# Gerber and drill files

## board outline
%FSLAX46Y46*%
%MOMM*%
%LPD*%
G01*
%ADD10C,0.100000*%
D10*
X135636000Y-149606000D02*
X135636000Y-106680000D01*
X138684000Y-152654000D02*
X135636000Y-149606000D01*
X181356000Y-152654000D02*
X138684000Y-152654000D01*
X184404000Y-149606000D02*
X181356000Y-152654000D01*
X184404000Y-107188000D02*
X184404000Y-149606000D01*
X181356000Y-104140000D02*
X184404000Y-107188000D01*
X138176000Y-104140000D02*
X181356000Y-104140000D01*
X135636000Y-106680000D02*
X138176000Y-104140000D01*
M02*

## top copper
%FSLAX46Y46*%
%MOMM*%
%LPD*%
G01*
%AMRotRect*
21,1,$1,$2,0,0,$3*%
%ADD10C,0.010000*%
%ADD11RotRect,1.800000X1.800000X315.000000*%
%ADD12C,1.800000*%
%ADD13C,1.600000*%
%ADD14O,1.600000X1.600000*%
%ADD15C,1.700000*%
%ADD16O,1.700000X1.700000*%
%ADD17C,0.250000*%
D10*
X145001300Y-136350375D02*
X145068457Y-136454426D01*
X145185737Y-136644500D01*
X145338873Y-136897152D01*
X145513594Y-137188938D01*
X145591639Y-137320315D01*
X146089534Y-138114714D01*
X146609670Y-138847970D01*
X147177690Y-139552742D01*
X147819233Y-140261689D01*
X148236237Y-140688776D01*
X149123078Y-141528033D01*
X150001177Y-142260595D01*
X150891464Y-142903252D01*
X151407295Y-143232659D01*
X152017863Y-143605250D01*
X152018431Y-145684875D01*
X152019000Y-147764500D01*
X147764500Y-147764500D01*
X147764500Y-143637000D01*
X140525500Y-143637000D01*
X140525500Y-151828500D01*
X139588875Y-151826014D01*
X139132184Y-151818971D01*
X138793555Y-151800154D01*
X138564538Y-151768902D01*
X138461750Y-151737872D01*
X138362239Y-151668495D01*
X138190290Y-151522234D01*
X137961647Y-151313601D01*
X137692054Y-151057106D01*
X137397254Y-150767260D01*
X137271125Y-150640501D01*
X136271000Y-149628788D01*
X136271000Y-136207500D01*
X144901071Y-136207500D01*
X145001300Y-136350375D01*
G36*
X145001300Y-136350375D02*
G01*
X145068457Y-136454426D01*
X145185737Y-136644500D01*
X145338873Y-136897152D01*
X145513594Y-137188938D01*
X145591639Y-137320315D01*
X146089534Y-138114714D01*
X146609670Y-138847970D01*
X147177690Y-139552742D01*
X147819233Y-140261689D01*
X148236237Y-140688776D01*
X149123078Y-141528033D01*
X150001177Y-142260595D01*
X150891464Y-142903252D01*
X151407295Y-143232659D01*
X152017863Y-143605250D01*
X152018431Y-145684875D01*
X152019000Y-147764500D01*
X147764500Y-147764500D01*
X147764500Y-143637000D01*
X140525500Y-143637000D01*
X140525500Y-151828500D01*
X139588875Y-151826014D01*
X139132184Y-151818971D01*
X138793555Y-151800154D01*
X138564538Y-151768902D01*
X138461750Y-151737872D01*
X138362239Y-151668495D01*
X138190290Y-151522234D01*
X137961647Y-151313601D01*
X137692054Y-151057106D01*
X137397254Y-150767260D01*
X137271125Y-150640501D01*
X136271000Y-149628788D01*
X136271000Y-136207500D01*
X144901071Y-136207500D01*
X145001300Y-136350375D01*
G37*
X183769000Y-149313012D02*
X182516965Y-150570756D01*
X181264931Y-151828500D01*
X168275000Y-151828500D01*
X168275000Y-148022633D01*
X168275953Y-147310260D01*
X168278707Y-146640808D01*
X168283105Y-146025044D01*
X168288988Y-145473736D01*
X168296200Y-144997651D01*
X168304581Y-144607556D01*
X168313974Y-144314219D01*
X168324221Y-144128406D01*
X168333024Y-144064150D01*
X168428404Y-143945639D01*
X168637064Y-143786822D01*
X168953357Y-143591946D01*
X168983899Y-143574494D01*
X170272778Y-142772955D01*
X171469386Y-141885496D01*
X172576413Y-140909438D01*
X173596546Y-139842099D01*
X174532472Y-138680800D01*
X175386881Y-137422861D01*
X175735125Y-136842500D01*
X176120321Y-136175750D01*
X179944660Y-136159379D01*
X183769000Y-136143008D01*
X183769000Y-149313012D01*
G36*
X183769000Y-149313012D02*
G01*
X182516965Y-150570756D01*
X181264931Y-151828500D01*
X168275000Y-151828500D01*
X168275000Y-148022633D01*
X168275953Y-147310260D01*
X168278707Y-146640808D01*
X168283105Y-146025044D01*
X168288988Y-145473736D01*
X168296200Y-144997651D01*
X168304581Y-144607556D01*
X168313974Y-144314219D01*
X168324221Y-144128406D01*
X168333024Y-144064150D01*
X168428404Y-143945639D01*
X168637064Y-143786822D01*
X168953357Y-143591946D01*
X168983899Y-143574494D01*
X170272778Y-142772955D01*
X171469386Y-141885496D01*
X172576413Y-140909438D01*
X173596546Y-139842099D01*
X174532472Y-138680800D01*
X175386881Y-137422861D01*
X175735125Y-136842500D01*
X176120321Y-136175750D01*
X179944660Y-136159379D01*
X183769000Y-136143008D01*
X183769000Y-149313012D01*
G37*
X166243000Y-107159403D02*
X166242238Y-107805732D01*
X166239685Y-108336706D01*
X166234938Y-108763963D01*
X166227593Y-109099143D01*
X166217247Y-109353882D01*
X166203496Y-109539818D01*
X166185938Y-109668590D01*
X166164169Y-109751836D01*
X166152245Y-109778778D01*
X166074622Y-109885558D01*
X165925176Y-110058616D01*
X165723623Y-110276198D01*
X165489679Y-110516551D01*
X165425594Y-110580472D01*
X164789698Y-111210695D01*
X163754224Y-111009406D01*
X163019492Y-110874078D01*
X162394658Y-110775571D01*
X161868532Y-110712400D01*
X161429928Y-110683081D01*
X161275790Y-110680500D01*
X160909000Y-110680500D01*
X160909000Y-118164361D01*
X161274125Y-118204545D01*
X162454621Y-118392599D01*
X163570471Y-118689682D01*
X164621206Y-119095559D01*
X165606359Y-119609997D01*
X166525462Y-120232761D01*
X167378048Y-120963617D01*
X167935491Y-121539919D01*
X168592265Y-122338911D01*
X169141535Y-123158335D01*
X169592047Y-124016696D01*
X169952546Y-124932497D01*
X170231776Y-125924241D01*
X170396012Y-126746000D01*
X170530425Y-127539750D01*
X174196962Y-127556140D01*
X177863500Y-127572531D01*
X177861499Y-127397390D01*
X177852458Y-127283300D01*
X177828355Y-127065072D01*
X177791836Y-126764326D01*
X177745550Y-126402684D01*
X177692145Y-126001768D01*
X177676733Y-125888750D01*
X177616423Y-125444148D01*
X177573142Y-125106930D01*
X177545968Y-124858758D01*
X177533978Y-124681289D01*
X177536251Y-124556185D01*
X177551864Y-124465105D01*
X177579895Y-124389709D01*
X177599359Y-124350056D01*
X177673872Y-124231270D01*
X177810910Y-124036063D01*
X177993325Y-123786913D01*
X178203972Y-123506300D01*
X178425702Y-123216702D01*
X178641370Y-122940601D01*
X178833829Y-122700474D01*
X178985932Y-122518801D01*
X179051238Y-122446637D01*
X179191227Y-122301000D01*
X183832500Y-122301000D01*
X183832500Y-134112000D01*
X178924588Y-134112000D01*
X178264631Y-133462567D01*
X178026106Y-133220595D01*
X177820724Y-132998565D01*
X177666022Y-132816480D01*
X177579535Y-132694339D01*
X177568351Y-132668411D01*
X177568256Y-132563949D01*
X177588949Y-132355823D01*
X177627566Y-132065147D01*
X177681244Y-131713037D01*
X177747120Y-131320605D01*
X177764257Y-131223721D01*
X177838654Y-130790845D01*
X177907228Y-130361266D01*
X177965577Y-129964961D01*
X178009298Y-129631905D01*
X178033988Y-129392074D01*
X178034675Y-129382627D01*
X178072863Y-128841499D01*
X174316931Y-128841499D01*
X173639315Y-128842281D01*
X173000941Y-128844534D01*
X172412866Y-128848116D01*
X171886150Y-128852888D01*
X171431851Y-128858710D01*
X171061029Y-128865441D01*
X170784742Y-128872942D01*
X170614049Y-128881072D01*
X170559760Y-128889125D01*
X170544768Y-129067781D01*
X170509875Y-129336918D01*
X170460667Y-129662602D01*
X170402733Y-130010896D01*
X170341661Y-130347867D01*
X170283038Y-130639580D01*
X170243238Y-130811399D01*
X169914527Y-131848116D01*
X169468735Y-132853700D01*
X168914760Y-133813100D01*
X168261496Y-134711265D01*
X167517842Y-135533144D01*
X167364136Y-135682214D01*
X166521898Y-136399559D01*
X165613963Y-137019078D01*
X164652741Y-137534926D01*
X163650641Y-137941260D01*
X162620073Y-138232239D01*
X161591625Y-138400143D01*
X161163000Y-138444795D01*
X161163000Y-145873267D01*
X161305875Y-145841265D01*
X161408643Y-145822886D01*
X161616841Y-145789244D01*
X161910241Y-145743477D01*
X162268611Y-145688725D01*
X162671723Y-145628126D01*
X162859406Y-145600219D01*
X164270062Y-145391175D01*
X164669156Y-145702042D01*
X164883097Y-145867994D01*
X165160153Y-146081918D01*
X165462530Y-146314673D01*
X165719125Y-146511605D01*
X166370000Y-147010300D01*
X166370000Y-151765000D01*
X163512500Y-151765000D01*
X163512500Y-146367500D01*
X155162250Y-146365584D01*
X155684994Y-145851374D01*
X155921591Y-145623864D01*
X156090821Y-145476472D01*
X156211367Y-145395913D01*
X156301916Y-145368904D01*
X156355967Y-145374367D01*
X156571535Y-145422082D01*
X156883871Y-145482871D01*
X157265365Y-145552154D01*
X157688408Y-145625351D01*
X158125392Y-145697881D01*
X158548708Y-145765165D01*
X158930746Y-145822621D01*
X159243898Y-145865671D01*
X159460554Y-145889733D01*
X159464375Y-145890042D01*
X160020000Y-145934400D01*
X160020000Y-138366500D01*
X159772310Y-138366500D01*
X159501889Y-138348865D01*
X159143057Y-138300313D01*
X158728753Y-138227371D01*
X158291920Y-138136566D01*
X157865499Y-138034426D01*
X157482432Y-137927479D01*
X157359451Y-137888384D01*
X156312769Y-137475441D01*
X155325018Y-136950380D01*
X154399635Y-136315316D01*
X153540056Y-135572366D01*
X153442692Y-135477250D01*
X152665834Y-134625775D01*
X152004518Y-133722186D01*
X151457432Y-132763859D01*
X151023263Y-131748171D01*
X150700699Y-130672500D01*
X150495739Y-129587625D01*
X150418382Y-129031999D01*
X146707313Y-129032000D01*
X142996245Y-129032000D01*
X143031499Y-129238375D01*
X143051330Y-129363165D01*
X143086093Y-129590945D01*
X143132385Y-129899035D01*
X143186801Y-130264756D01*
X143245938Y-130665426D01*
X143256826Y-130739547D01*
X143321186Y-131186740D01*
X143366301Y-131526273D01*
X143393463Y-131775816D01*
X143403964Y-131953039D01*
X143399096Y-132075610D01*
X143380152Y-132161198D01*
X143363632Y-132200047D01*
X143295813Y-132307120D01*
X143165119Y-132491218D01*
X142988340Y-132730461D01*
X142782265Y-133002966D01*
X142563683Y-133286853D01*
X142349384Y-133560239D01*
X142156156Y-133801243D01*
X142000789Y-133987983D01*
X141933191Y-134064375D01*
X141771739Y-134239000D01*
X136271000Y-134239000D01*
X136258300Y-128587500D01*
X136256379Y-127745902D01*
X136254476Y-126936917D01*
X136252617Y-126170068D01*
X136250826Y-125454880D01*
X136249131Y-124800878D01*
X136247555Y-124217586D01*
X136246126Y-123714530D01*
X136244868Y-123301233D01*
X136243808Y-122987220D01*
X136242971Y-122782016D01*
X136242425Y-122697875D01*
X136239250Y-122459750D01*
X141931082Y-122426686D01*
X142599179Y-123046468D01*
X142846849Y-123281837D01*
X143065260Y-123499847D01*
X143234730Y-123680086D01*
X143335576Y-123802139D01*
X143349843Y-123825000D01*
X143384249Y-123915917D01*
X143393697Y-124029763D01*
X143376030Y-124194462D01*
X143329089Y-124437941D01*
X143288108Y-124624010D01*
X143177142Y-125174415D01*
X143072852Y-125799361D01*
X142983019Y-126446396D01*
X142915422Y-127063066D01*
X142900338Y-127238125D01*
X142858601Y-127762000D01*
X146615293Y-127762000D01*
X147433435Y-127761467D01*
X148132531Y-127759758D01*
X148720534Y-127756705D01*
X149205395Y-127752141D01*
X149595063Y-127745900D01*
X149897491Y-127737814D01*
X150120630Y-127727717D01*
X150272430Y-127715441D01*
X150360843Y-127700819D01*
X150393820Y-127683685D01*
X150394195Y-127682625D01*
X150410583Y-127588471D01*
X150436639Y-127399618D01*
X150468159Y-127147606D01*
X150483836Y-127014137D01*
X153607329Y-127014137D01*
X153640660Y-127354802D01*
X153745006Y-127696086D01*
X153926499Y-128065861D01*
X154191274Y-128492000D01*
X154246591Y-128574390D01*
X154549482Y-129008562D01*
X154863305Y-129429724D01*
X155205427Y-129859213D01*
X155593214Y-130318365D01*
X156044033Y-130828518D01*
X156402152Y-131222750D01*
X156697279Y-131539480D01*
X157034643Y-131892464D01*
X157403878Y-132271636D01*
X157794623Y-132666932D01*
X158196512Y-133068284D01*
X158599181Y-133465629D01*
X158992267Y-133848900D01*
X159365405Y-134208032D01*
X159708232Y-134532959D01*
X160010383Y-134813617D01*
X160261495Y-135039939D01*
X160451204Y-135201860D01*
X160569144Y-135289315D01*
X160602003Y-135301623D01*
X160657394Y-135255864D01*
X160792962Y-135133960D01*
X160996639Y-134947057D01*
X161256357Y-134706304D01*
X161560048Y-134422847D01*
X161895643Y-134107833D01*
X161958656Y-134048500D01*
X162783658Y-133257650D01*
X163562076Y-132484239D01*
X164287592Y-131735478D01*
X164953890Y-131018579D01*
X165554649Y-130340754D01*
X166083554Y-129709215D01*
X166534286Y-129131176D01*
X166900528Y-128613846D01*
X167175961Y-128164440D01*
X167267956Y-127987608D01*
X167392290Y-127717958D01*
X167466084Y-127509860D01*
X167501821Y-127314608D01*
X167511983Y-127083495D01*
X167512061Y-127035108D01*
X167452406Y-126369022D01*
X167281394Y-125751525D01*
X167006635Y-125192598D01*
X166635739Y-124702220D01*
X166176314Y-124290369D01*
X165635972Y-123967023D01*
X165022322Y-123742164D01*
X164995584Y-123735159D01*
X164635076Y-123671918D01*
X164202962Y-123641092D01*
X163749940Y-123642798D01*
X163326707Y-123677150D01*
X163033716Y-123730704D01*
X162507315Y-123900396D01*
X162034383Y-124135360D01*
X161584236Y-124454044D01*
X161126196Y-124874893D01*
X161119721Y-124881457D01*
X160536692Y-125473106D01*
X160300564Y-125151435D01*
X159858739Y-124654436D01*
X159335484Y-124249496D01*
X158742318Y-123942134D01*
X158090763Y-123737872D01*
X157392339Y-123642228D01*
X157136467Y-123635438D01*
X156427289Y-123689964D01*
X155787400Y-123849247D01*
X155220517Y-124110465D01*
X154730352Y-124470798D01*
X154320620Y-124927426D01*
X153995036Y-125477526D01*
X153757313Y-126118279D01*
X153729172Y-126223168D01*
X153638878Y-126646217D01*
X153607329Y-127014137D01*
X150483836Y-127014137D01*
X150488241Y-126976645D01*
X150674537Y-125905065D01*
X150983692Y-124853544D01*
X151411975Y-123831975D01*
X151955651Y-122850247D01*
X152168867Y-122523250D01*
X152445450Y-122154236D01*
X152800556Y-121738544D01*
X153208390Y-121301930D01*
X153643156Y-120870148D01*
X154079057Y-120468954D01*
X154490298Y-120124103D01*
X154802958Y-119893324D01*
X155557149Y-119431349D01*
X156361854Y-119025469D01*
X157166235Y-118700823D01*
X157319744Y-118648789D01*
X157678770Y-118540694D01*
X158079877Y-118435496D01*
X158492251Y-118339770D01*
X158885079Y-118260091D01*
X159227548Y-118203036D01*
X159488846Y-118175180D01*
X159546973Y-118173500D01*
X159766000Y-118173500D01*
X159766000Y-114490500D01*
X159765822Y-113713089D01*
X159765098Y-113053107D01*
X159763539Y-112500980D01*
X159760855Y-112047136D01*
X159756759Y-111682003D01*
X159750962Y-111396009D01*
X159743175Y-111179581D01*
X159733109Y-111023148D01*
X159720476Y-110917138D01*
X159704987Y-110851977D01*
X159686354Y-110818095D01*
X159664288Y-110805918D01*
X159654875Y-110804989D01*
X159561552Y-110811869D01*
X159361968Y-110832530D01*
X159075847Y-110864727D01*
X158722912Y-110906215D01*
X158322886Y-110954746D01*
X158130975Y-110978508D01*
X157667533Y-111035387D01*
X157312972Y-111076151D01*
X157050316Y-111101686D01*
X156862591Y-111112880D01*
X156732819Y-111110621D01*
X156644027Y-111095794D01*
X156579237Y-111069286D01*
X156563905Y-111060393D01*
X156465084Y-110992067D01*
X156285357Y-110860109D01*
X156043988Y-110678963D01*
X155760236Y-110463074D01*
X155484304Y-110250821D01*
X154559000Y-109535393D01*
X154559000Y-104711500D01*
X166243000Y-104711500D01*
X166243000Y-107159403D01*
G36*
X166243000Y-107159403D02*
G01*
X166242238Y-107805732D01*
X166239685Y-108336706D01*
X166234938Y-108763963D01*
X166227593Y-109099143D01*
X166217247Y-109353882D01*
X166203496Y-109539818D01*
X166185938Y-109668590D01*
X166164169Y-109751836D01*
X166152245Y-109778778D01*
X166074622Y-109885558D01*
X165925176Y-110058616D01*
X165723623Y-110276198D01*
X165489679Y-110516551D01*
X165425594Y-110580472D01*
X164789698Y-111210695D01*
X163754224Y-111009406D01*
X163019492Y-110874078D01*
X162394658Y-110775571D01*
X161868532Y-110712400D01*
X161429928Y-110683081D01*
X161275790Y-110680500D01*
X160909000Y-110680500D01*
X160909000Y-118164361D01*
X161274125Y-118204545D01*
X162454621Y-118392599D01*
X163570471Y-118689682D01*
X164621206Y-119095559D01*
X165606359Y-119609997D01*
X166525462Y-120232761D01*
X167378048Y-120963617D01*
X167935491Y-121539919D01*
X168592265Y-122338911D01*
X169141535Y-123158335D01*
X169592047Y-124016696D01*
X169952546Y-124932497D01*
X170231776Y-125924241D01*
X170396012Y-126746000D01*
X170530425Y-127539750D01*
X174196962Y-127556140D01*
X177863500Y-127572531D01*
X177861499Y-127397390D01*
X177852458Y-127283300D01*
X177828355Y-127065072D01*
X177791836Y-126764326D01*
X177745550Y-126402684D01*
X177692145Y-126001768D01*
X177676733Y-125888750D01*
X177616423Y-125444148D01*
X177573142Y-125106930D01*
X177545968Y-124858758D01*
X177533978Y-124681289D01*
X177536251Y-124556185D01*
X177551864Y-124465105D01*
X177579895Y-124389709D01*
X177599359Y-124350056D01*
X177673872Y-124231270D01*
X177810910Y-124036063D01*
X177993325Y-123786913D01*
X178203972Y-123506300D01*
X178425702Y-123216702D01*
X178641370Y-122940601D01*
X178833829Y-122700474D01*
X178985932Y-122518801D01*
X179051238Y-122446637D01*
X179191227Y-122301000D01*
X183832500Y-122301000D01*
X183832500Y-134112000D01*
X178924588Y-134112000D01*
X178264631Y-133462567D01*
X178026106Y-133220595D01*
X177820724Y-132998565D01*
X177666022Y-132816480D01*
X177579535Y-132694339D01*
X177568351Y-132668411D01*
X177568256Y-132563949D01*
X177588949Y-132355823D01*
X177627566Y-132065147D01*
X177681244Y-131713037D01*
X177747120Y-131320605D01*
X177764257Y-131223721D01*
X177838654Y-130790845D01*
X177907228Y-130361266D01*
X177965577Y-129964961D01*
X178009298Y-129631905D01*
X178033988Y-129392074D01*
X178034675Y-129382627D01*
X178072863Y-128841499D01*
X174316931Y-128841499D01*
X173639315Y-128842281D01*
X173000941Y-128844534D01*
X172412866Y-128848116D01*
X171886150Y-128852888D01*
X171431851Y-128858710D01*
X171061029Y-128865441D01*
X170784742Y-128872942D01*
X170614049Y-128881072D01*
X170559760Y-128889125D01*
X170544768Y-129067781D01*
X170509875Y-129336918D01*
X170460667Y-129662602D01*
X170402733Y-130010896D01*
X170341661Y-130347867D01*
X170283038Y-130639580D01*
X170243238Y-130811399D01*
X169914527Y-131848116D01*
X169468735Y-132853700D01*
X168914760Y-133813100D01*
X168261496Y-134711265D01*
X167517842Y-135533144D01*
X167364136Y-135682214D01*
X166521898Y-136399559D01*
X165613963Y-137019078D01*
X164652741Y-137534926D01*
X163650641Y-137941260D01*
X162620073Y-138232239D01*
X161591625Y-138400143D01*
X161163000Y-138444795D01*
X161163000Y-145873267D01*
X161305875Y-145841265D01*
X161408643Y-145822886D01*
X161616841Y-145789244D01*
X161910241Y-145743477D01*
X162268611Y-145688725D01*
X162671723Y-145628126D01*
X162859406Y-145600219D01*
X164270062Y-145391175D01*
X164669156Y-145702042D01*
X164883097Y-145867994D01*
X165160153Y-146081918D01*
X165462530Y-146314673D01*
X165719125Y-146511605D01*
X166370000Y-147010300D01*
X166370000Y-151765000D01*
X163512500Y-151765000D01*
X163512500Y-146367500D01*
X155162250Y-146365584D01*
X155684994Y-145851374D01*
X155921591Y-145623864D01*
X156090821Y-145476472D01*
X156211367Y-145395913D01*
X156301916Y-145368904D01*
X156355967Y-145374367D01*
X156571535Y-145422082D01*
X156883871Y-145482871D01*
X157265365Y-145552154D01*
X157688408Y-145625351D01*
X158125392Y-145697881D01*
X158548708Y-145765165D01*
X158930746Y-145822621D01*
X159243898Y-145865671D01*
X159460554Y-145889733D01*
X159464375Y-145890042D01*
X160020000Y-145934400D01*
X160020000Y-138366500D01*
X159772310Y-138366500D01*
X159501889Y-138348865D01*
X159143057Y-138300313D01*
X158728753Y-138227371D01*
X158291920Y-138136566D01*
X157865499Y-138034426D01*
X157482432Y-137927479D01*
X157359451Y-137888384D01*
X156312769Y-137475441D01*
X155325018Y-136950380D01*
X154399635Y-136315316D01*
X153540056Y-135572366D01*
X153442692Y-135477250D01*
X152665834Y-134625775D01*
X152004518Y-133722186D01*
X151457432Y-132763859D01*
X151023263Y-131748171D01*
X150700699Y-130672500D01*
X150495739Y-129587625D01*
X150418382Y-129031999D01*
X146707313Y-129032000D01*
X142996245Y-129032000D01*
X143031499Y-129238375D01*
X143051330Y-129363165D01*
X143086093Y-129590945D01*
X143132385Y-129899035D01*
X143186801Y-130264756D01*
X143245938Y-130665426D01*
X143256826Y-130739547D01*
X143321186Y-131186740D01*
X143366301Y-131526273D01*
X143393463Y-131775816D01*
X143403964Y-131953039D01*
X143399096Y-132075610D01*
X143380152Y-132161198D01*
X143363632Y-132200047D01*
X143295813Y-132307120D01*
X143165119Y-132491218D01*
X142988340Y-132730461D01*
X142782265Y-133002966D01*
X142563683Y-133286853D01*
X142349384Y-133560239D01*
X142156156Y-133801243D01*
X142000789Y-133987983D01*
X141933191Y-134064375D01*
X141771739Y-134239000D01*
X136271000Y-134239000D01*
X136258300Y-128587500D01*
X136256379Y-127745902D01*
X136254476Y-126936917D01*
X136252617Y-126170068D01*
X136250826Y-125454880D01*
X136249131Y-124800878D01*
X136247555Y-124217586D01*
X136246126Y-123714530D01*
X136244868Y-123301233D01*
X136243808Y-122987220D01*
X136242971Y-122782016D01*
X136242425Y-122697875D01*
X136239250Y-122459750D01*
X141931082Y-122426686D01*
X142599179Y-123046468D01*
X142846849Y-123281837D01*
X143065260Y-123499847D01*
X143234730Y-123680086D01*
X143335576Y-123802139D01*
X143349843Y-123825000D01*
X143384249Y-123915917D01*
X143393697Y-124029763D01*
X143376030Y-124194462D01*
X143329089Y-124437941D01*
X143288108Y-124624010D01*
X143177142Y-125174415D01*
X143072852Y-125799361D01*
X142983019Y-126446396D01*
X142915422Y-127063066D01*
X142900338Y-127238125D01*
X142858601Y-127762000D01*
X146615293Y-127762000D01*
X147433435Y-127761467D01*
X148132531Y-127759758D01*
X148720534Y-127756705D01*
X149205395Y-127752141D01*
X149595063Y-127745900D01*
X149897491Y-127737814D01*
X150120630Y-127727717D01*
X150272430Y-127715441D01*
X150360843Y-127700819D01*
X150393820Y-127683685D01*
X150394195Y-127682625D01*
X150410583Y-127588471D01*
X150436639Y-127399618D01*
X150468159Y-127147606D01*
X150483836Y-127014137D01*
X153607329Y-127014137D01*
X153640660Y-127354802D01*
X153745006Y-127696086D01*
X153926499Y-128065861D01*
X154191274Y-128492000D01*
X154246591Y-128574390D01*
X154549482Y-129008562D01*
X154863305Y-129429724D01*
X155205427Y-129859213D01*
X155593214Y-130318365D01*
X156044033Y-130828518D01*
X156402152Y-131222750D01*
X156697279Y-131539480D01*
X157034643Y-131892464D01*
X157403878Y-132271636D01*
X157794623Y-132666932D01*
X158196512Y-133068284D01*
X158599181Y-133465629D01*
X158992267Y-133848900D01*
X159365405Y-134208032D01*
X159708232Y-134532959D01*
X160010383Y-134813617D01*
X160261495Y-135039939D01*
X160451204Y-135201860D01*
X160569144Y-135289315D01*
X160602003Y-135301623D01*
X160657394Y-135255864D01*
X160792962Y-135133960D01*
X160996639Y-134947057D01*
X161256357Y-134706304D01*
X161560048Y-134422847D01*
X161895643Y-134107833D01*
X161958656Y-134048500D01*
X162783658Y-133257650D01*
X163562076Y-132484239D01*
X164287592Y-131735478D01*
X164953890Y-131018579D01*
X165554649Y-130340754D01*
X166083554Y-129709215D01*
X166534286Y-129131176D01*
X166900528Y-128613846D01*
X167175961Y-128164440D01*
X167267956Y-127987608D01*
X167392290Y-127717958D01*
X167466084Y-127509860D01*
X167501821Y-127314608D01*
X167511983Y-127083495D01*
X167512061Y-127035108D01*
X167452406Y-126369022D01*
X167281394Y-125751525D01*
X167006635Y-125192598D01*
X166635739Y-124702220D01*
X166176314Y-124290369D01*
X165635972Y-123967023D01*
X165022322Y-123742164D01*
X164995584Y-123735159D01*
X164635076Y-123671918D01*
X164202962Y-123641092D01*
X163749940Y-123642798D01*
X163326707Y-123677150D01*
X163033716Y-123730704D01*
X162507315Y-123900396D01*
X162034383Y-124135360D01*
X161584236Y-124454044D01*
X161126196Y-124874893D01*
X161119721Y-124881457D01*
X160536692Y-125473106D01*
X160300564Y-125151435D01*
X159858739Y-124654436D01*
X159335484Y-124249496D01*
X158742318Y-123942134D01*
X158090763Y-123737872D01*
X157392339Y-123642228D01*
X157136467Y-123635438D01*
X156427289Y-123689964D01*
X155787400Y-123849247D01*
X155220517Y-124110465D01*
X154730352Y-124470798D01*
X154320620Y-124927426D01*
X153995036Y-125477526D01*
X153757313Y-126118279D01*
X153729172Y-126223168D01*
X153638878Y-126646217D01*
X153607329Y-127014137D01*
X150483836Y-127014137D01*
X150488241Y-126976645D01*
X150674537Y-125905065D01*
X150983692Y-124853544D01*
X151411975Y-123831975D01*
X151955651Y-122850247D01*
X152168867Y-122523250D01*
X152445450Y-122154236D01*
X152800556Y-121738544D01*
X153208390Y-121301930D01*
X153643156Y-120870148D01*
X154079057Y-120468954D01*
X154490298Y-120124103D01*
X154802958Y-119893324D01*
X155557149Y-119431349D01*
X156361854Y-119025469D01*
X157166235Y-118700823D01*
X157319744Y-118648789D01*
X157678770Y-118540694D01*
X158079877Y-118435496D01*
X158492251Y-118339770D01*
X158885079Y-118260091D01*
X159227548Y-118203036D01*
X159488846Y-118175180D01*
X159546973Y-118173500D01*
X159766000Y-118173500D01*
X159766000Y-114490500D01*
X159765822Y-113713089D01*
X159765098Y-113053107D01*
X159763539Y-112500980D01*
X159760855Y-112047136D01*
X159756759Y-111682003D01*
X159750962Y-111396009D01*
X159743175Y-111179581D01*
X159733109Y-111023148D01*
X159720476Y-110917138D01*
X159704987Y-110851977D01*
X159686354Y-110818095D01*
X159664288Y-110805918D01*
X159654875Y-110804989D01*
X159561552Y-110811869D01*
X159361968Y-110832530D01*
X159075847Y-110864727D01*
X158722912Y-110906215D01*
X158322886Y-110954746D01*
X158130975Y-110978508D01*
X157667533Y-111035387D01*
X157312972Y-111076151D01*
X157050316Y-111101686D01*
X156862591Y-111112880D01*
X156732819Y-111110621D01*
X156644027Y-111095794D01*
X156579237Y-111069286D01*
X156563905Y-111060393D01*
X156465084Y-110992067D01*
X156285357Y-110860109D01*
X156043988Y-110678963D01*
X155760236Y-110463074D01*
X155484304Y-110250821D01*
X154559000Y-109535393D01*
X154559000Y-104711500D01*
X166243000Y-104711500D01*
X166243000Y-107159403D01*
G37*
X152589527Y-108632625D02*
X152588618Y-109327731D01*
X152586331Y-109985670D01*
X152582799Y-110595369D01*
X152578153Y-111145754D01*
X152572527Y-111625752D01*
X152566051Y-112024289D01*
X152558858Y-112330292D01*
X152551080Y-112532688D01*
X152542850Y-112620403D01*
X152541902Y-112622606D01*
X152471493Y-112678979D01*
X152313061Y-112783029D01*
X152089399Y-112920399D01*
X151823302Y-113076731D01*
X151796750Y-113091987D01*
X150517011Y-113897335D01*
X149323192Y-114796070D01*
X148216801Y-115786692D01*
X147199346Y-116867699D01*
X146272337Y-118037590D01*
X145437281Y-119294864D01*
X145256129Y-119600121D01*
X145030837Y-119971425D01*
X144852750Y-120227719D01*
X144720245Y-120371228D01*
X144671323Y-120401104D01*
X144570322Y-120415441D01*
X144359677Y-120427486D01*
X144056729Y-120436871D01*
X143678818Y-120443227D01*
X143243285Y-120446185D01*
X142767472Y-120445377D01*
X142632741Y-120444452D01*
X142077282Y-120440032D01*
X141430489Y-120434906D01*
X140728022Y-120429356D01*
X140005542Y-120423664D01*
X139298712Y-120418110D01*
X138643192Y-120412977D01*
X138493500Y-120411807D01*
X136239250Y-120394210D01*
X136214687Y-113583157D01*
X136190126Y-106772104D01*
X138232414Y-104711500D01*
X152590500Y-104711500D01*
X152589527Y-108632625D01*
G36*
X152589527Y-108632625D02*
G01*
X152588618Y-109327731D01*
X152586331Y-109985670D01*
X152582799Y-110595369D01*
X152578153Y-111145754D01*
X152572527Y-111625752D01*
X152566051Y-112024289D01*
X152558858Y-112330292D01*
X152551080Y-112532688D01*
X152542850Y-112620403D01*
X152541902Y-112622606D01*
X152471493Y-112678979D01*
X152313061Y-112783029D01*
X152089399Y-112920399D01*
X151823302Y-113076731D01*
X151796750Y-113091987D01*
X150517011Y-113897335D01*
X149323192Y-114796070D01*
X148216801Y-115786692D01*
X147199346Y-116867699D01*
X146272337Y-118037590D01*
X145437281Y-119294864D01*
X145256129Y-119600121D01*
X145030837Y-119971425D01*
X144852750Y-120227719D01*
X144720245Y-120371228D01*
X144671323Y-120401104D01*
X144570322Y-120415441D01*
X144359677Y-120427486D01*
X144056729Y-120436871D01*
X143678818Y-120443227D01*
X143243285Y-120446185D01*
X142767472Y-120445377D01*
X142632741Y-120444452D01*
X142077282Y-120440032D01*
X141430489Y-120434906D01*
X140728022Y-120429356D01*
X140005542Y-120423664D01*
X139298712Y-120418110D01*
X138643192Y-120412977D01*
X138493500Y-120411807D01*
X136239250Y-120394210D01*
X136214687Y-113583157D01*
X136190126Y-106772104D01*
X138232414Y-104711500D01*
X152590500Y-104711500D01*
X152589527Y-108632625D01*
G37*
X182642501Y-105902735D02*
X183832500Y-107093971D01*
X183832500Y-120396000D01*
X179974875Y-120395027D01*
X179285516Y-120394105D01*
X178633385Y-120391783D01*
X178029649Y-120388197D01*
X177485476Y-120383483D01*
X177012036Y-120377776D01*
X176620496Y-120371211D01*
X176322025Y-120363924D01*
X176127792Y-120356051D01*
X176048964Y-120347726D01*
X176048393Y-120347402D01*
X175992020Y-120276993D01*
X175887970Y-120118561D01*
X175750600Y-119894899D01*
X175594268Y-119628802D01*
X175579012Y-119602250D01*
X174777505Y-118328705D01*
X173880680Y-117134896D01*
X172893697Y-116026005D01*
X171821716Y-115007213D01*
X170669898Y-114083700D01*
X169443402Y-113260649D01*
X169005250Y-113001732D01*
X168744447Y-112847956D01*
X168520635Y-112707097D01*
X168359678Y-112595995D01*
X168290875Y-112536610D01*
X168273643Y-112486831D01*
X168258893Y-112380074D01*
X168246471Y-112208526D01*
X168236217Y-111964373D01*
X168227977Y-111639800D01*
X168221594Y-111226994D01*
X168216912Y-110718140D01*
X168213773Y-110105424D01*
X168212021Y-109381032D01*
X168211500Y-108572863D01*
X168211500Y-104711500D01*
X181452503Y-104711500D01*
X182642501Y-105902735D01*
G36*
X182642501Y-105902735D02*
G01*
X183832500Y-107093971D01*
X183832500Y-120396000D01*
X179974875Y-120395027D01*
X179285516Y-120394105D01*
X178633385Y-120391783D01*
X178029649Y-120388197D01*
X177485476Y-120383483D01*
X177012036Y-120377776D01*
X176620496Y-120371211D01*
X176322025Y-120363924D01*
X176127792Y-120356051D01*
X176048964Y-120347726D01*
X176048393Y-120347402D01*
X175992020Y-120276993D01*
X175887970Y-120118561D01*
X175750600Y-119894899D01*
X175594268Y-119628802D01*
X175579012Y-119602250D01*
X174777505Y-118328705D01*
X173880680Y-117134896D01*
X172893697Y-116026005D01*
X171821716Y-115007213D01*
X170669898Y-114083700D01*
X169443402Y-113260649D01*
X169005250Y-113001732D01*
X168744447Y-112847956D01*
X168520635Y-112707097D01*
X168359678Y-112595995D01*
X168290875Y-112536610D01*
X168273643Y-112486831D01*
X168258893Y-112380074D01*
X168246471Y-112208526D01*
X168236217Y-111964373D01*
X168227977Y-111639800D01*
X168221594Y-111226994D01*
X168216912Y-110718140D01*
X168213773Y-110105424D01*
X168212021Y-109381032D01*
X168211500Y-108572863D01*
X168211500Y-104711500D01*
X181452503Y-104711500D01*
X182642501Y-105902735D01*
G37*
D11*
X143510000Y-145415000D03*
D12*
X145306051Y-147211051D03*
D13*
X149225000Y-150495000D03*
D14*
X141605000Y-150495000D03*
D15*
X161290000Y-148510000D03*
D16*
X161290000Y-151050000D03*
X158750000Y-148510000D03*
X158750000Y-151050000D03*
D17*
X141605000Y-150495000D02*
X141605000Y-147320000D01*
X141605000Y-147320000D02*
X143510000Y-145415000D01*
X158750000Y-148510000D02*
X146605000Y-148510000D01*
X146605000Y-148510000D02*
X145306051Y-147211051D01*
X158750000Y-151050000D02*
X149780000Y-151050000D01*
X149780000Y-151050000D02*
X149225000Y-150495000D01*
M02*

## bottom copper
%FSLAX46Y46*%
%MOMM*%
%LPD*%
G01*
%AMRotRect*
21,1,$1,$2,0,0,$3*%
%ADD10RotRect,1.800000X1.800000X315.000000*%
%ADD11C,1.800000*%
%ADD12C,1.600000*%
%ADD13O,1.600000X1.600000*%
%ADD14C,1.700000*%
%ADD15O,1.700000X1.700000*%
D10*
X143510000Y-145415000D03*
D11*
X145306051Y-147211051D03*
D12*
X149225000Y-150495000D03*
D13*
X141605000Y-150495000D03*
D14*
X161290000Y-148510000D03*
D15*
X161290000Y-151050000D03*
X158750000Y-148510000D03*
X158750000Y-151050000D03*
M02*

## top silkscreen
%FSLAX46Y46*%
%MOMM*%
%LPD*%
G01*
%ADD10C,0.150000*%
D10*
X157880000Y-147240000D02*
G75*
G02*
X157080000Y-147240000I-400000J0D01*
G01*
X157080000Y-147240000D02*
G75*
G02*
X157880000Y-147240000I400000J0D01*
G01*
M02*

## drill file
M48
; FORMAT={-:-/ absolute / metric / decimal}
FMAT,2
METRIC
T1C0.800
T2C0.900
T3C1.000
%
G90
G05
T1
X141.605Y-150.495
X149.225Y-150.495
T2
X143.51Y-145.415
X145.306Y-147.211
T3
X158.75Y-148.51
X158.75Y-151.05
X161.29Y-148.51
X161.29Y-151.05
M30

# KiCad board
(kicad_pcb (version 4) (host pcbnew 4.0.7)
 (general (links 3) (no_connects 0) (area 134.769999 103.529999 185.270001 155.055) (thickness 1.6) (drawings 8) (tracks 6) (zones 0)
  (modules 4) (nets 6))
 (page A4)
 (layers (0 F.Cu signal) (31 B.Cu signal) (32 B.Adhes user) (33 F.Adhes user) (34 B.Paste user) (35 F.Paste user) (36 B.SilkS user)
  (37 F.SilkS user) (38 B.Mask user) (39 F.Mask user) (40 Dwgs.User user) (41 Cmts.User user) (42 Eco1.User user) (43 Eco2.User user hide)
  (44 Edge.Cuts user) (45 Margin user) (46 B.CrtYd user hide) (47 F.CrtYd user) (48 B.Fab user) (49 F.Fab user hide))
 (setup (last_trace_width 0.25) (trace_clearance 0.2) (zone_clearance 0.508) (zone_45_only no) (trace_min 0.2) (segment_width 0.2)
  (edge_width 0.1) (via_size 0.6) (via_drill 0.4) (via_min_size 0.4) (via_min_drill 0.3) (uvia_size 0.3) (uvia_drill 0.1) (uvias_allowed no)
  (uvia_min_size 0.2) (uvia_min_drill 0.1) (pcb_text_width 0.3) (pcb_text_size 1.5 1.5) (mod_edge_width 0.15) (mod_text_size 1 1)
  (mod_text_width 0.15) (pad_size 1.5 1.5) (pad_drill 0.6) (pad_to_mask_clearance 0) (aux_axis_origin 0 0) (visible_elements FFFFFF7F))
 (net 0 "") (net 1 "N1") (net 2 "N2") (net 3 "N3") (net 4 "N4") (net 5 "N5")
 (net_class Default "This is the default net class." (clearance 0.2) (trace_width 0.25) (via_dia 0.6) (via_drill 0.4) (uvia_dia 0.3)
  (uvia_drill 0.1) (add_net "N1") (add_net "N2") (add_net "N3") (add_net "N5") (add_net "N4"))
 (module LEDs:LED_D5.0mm (layer B.Cu) (at 143.51 145.415 315)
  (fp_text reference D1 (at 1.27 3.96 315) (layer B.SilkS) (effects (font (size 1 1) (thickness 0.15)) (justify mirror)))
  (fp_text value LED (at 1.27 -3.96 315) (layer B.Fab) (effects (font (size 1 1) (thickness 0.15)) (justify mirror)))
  (pad 1 thru_hole rect (at 0 0 315) (size 1.8 1.8) (drill 0.9) (layers *.Cu *.Mask) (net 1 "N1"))
  (pad 2 thru_hole circle (at 2.54 0 315) (size 1.8 1.8) (drill 0.9) (layers *.Cu *.Mask) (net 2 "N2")))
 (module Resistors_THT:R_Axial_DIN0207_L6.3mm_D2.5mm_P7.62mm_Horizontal (layer B.Cu) (at 149.225 150.495 180)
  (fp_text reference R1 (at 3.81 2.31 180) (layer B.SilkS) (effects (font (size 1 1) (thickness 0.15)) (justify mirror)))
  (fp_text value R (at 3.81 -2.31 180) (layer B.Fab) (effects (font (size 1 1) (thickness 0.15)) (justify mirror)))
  (pad 1 thru_hole circle (at 0 0 180) (size 1.6 1.6) (drill 0.8) (layers *.Cu *.Mask) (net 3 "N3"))
  (pad 2 thru_hole oval (at 7.62 0 180) (size 1.6 1.6) (drill 0.8) (layers *.Cu *.Mask) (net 1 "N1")))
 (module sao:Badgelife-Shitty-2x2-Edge (layer F.Cu) (at 160.02 144.78)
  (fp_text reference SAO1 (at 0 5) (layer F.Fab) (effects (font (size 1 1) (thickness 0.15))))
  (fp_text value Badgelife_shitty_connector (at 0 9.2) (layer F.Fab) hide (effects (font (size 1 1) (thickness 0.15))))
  (fp_circle (center -2.54 2.46) (end -2.14 2.46) (layer F.SilkS) (width 0.15))
  (pad 4 thru_hole circle (at 1.27 3.73) (size 1.7 1.7) (drill 1) (layers *.Cu *.Mask) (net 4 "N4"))
  (pad 3 thru_hole oval (at 1.27 6.27) (size 1.7 1.7) (drill 1) (layers *.Cu *.Mask) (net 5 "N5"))
  (pad 1 thru_hole oval (at -1.27 3.73) (size 1.7 1.7) (drill 1) (layers *.Cu *.Mask) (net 2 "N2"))
  (pad 2 thru_hole oval (at -1.27 6.27) (size 1.7 1.7) (drill 1) (layers *.Cu *.Mask) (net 3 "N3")))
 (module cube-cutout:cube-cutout (layer F.Cu) (at 160.02 128.27)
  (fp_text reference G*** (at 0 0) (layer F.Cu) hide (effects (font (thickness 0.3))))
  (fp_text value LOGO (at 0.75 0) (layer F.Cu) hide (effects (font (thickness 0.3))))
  (fp_poly
   (pts (xy -15.0187 8.080375) (xy -14.951543 8.184426) (xy -14.834263 8.3745) (xy -14.681127 8.627152) (xy -14.506406 8.918938)
    (xy -14.428361 9.050315) (xy -13.930466 9.844714) (xy -13.41033 10.57797) (xy -12.84231 11.282742) (xy -12.200767 11.991689)
    (xy -11.783763 12.418776) (xy -10.896922 13.258033) (xy -10.018823 13.990595) (xy -9.128536 14.633252) (xy -8.612705 14.962659)
    (xy -8.002137 15.33525) (xy -8.001569 17.414875) (xy -8.001 19.4945) (xy -12.2555 19.4945) (xy -12.2555 15.367) (xy -19.4945 15.367)
    (xy -19.4945 23.5585) (xy -20.431125 23.556014) (xy -20.887816 23.548971) (xy -21.226445 23.530154) (xy -21.455462 23.498902)
    (xy -21.55825 23.467872) (xy -21.657761 23.398495) (xy -21.82971 23.252234) (xy -22.058353 23.043601) (xy -22.327946 22.787106)
    (xy -22.622746 22.49726) (xy -22.748875 22.370501) (xy -23.749 21.358788) (xy -23.749 7.9375) (xy -15.118929 7.9375)
    (xy -15.0187 8.080375))
   (layer F.Cu) (width 0.01))
  (fp_poly
   (pts (xy 23.749 21.043012) (xy 22.496965 22.300756) (xy 21.244931 23.5585) (xy 8.255 23.5585) (xy 8.255 19.752633) (xy 8.255953 19.04026)
    (xy 8.258707 18.370808) (xy 8.263105 17.755044) (xy 8.268988 17.203736) (xy 8.2762 16.727651) (xy 8.284581 16.337556)
    (xy 8.293974 16.044219) (xy 8.304221 15.858406) (xy 8.313024 15.79415) (xy 8.408404 15.675639) (xy 8.617064 15.516822)
    (xy 8.933357 15.321946) (xy 8.963899 15.304494) (xy 10.252778 14.502955) (xy 11.449386 13.615496) (xy 12.556413 12.639438)
    (xy 13.576546 11.572099) (xy 14.512472 10.4108) (xy 15.366881 9.152861) (xy 15.715125 8.5725) (xy 16.100321 7.90575)
    (xy 19.92466 7.889379) (xy 23.749 7.873008) (xy 23.749 21.043012))
   (layer F.Cu) (width 0.01))
  (fp_poly
   (pts (xy 6.223 -21.110597) (xy 6.222238 -20.464268) (xy 6.219685 -19.933294) (xy 6.214938 -19.506037) (xy 6.207593 -19.170857)
    (xy 6.197247 -18.916118) (xy 6.183496 -18.730182) (xy 6.165938 -18.60141) (xy 6.144169 -18.518164) (xy 6.132245 -18.491222)
    (xy 6.054622 -18.384442) (xy 5.905176 -18.211384) (xy 5.703623 -17.993802) (xy 5.469679 -17.753449) (xy 5.405594 -17.689528)
    (xy 4.769698 -17.059305) (xy 3.734224 -17.260594) (xy 2.999492 -17.395922) (xy 2.374658 -17.494429) (xy 1.848532 -17.5576)
    (xy 1.409928 -17.586919) (xy 1.25579 -17.5895) (xy 0.889 -17.5895) (xy 0.889 -10.105639) (xy 1.254125 -10.065455)
    (xy 2.434621 -9.877401) (xy 3.550471 -9.580318) (xy 4.601206 -9.174441) (xy 5.586359 -8.660003) (xy 6.505462 -8.037239)
    (xy 7.358048 -7.306383) (xy 7.915491 -6.730081) (xy 8.572265 -5.931089) (xy 9.121535 -5.111665) (xy 9.572047 -4.253304)
    (xy 9.932546 -3.337503) (xy 10.211776 -2.345759) (xy 10.376012 -1.524) (xy 10.510425 -0.73025) (xy 14.176962 -0.71386)
    (xy 17.8435 -0.697469) (xy 17.841499 -0.87261) (xy 17.832458 -0.9867) (xy 17.808355 -1.204928) (xy 17.771836 -1.505674)
    (xy 17.72555 -1.867316) (xy 17.672145 -2.268232) (xy 17.656733 -2.38125) (xy 17.596423 -2.825852) (xy 17.553142 -3.16307)
    (xy 17.525968 -3.411242) (xy 17.513978 -3.588711) (xy 17.516251 -3.713815) (xy 17.531864 -3.804895) (xy 17.559895 -3.880291)
    (xy 17.579359 -3.919944) (xy 17.653872 -4.03873) (xy 17.79091 -4.233937) (xy 17.973325 -4.483087) (xy 18.183972 -4.7637)
    (xy 18.405702 -5.053298) (xy 18.62137 -5.329399) (xy 18.813829 -5.569526) (xy 18.965932 -5.751199) (xy 19.031238 -5.823363)
    (xy 19.171227 -5.969) (xy 23.8125 -5.969) (xy 23.8125 5.842) (xy 18.904588 5.842) (xy 18.244631 5.192567) (xy 18.006106 4.950595)
    (xy 17.800724 4.728565) (xy 17.646022 4.54648) (xy 17.559535 4.424339) (xy 17.548351 4.398411) (xy 17.548256 4.293949)
    (xy 17.568949 4.085823) (xy 17.607566 3.795147) (xy 17.661244 3.443037) (xy 17.72712 3.050605) (xy 17.744257 2.953721)
    (xy 17.818654 2.520845) (xy 17.887228 2.091266) (xy 17.945577 1.694961) (xy 17.989298 1.361905) (xy 18.013988 1.122074)
    (xy 18.014675 1.112627) (xy 18.052863 0.571499) (xy 14.296931 0.571499) (xy 13.619315 0.572281) (xy 12.980941 0.574534)
    (xy 12.392866 0.578116) (xy 11.86615 0.582888) (xy 11.411851 0.58871) (xy 11.041029 0.595441) (xy 10.764742 0.602942)
    (xy 10.594049 0.611072) (xy 10.53976 0.619125) (xy 10.524768 0.797781) (xy 10.489875 1.066918) (xy 10.440667 1.392602)
    (xy 10.382733 1.740896) (xy 10.321661 2.077867) (xy 10.263038 2.36958) (xy 10.223238 2.541399) (xy 9.894527 3.578116)
    (xy 9.448735 4.5837) (xy 8.89476 5.5431) (xy 8.241496 6.441265) (xy 7.497842 7.263144) (xy 7.344136 7.412214) (xy 6.501898 8.129559)
    (xy 5.593963 8.749078) (xy 4.632741 9.264926) (xy 3.630641 9.67126) (xy 2.600073 9.962239) (xy 1.571625 10.130143) (xy 1.143 10.174795)
    (xy 1.143 17.603267) (xy 1.285875 17.571265) (xy 1.388643 17.552886) (xy 1.596841 17.519244) (xy 1.890241 17.473477)
    (xy 2.248611 17.418725) (xy 2.651723 17.358126) (xy 2.839406 17.330219) (xy 4.250062 17.121175) (xy 4.649156 17.432042)
    (xy 4.863097 17.597994) (xy 5.140153 17.811918) (xy 5.44253 18.044673) (xy 5.699125 18.241605) (xy 6.35 18.7403) (xy 6.35 23.495)
    (xy 3.4925 23.495) (xy 3.4925 18.0975) (xy -4.85775 18.095584) (xy -4.335006 17.581374) (xy -4.098409 17.353864)
    (xy -3.929179 17.206472) (xy -3.808633 17.125913) (xy -3.718084 17.098904) (xy -3.664033 17.104367) (xy -3.448465 17.152082)
    (xy -3.136129 17.212871) (xy -2.754635 17.282154) (xy -2.331592 17.355351) (xy -1.894608 17.427881) (xy -1.471292 17.495165)
    (xy -1.089254 17.552621) (xy -0.776102 17.595671) (xy -0.559446 17.619733) (xy -0.555625 17.620042) (xy 0 17.6644) (xy 0 10.0965)
    (xy -0.24769 10.0965) (xy -0.518111 10.078865) (xy -0.876943 10.030313) (xy -1.291247 9.957371) (xy -1.72808 9.866566)
    (xy -2.154501 9.764426) (xy -2.537568 9.657479) (xy -2.660549 9.618384) (xy -3.707231 9.205441) (xy -4.694982 8.68038)
    (xy -5.620365 8.045316) (xy -6.479944 7.302366) (xy -6.577308 7.20725) (xy -7.354166 6.355775) (xy -8.015482 5.452186)
    (xy -8.562568 4.493859) (xy -8.996737 3.478171) (xy -9.319301 2.4025) (xy -9.524261 1.317625) (xy -9.601618 0.761999)
    (xy -13.312687 0.762) (xy -17.023755 0.762) (xy -16.988501 0.968375) (xy -16.96867 1.093165) (xy -16.933907 1.320945)
    (xy -16.887615 1.629035) (xy -16.833199 1.994756) (xy -16.774062 2.395426) (xy -16.763174 2.469547) (xy -16.698814 2.91674)
    (xy -16.653699 3.256273) (xy -16.626537 3.505816) (xy -16.616036 3.683039) (xy -16.620904 3.80561) (xy -16.639848 3.891198)
    (xy -16.656368 3.930047) (xy -16.724187 4.03712) (xy -16.854881 4.221218) (xy -17.03166 4.460461) (xy -17.237735 4.732966)
    (xy -17.456317 5.016853) (xy -17.670616 5.290239) (xy -17.863844 5.531243) (xy -18.019211 5.717983) (xy -18.086809 5.794375)
    (xy -18.248261 5.969) (xy -23.749 5.969) (xy -23.7617 0.3175) (xy -23.763621 -0.524098) (xy -23.765524 -1.333083)
    (xy -23.767383 -2.099932) (xy -23.769174 -2.81512) (xy -23.770869 -3.469122) (xy -23.772445 -4.052414) (xy -23.773874 -4.55547)
    (xy -23.775132 -4.968767) (xy -23.776192 -5.28278) (xy -23.777029 -5.487984) (xy -23.777575 -5.572125) (xy -23.78075 -5.81025)
    (xy -18.088918 -5.843314) (xy -17.420821 -5.223532) (xy -17.173151 -4.988163) (xy -16.95474 -4.770153) (xy -16.78527 -4.589914)
    (xy -16.684424 -4.467861) (xy -16.670157 -4.445) (xy -16.635751 -4.354083) (xy -16.626303 -4.240237) (xy -16.64397 -4.075538)
    (xy -16.690911 -3.832059) (xy -16.731892 -3.64599) (xy -16.842858 -3.095585) (xy -16.947148 -2.470639) (xy -17.036981 -1.823604)
    (xy -17.104578 -1.206934) (xy -17.119662 -1.031875) (xy -17.161399 -0.508) (xy -13.404707 -0.508) (xy -12.586565 -0.508533)
    (xy -11.887469 -0.510242) (xy -11.299466 -0.513295) (xy -10.814605 -0.517859) (xy -10.424937 -0.5241) (xy -10.122509 -0.532186)
    (xy -9.89937 -0.542283) (xy -9.74757 -0.554559) (xy -9.659157 -0.569181) (xy -9.62618 -0.586315) (xy -9.625805 -0.587375)
    (xy -9.609417 -0.681529) (xy -9.583361 -0.870382) (xy -9.551841 -1.122394) (xy -9.536164 -1.255863) (xy -6.412671 -1.255863)
    (xy -6.37934 -0.915198) (xy -6.274994 -0.573914) (xy -6.093501 -0.204139) (xy -5.828726 0.222) (xy -5.773409 0.30439)
    (xy -5.470518 0.738562) (xy -5.156695 1.159724) (xy -4.814573 1.589213) (xy -4.426786 2.048365) (xy -3.975967 2.558518)
    (xy -3.617848 2.95275) (xy -3.322721 3.26948) (xy -2.985357 3.622464) (xy -2.616122 4.001636) (xy -2.225377 4.396932)
    (xy -1.823488 4.798284) (xy -1.420819 5.195629) (xy -1.027733 5.5789) (xy -0.654595 5.938032) (xy -0.311768 6.262959)
    (xy -0.009617 6.543617) (xy 0.241495 6.769939) (xy 0.431204 6.93186) (xy 0.549144 7.019315) (xy 0.582003 7.031623)
    (xy 0.637394 6.985864) (xy 0.772962 6.86396) (xy 0.976639 6.677057) (xy 1.236357 6.436304) (xy 1.540048 6.152847) (xy 1.875643 5.837833)
    (xy 1.938656 5.7785) (xy 2.763658 4.98765) (xy 3.542076 4.214239) (xy 4.267592 3.465478) (xy 4.93389 2.748579) (xy 5.534649 2.070754)
    (xy 6.063554 1.439215) (xy 6.514286 0.861176) (xy 6.880528 0.343846) (xy 7.155961 -0.10556) (xy 7.247956 -0.282392)
    (xy 7.37229 -0.552042) (xy 7.446084 -0.76014) (xy 7.481821 -0.955392) (xy 7.491983 -1.186505) (xy 7.492061 -1.234892)
    (xy 7.432406 -1.900978) (xy 7.261394 -2.518475) (xy 6.986635 -3.077402) (xy 6.615739 -3.56778) (xy 6.156314 -3.979631)
    (xy 5.615972 -4.302977) (xy 5.002322 -4.527836) (xy 4.975584 -4.534841) (xy 4.615076 -4.598082) (xy 4.182962 -4.628908)
    (xy 3.72994 -4.627202) (xy 3.306707 -4.59285) (xy 3.013716 -4.539296) (xy 2.487315 -4.369604) (xy 2.014383 -4.13464)
    (xy 1.564236 -3.815956) (xy 1.106196 -3.395107) (xy 1.099721 -3.388543) (xy 0.516692 -2.796894) (xy 0.280564 -3.118565)
    (xy -0.161261 -3.615564) (xy -0.684516 -4.020504) (xy -1.277682 -4.327866) (xy -1.929237 -4.532128) (xy -2.627661 -4.627772)
    (xy -2.883533 -4.634562) (xy -3.592711 -4.580036) (xy -4.2326 -4.420753) (xy -4.799483 -4.159535) (xy -5.289648 -3.799202)
    (xy -5.69938 -3.342574) (xy -6.024964 -2.792474) (xy -6.262687 -2.151721) (xy -6.290828 -2.046832) (xy -6.381122 -1.623783)
    (xy -6.412671 -1.255863) (xy -9.536164 -1.255863) (xy -9.531759 -1.293355) (xy -9.345463 -2.364935) (xy -9.036308 -3.416456)
    (xy -8.608025 -4.438025) (xy -8.064349 -5.419753) (xy -7.851133 -5.74675) (xy -7.57455 -6.115764) (xy -7.219444 -6.531456)
    (xy -6.81161 -6.96807) (xy -6.376844 -7.399852) (xy -5.940943 -7.801046) (xy -5.529702 -8.145897) (xy -5.217042 -8.376676)
    (xy -4.462851 -8.838651) (xy -3.658146 -9.244531) (xy -2.853765 -9.569177) (xy -2.700256 -9.621211) (xy -2.34123 -9.729306)
    (xy -1.940123 -9.834504) (xy -1.527749 -9.93023) (xy -1.134921 -10.009909) (xy -0.792452 -10.066964) (xy -0.531154 -10.09482)
    (xy -0.473027 -10.0965) (xy -0.254 -10.0965) (xy -0.254 -13.7795) (xy -0.254178 -14.556911) (xy -0.254902 -15.216893)
    (xy -0.256461 -15.76902) (xy -0.259145 -16.222864) (xy -0.263241 -16.587997) (xy -0.269038 -16.873991) (xy -0.276825 -17.090419)
    (xy -0.286891 -17.246852) (xy -0.299524 -17.352862) (xy -0.315013 -17.418023) (xy -0.333646 -17.451905) (xy -0.355712 -17.464082)
    (xy -0.365125 -17.465011) (xy -0.458448 -17.458131) (xy -0.658032 -17.43747) (xy -0.944153 -17.405273) (xy -1.297088 -17.363785)
    (xy -1.697114 -17.315254) (xy -1.889025 -17.291492) (xy -2.352467 -17.234613) (xy -2.707028 -17.193849) (xy -2.969684 -17.168314)
    (xy -3.157409 -17.15712) (xy -3.287181 -17.159379) (xy -3.375973 -17.174206) (xy -3.440763 -17.200714) (xy -3.456095 -17.209607)
    (xy -3.554916 -17.277933) (xy -3.734643 -17.409891) (xy -3.976012 -17.591037) (xy -4.259764 -17.806926) (xy -4.535696 -18.019179)
    (xy -5.461 -18.734607) (xy -5.461 -23.5585) (xy 6.223 -23.5585) (xy 6.223 -21.110597))
   (layer F.Cu) (width 0.01))
  (fp_poly
   (pts (xy -7.430473 -19.637375) (xy -7.431382 -18.942269) (xy -7.433669 -18.28433) (xy -7.437201 -17.674631) (xy -7.441847 -17.124246)
    (xy -7.447473 -16.644248) (xy -7.453949 -16.245711) (xy -7.461142 -15.939708) (xy -7.46892 -15.737312) (xy -7.47715 -15.649597)
    (xy -7.478098 -15.647394) (xy -7.548507 -15.591021) (xy -7.706939 -15.486971) (xy -7.930601 -15.349601) (xy -8.196698 -15.193269)
    (xy -8.22325 -15.178013) (xy -9.502989 -14.372665) (xy -10.696808 -13.47393) (xy -11.803199 -12.483308) (xy -12.820654 -11.402301)
    (xy -13.747663 -10.23241) (xy -14.582719 -8.975136) (xy -14.763871 -8.669879) (xy -14.989163 -8.298575) (xy -15.16725 -8.042281)
    (xy -15.299755 -7.898772) (xy -15.348677 -7.868896) (xy -15.449678 -7.854559) (xy -15.660323 -7.842514) (xy -15.963271 -7.833129)
    (xy -16.341182 -7.826773) (xy -16.776715 -7.823815) (xy -17.252528 -7.824623) (xy -17.387259 -7.825548) (xy -17.942718 -7.829968)
    (xy -18.589511 -7.835094) (xy -19.291978 -7.840644) (xy -20.014458 -7.846336) (xy -20.721288 -7.85189) (xy -21.376808 -7.857023)
    (xy -21.5265 -7.858193) (xy -23.78075 -7.87579) (xy -23.805313 -14.686843) (xy -23.829874 -21.497896) (xy -21.787586 -23.5585)
    (xy -7.4295 -23.5585) (xy -7.430473 -19.637375))
   (layer F.Cu) (width 0.01))
  (fp_poly
   (pts (xy 22.622501 -22.367265) (xy 23.8125 -21.176029) (xy 23.8125 -7.874) (xy 19.954875 -7.874973) (xy 19.265516 -7.875895)
    (xy 18.613385 -7.878217) (xy 18.009649 -7.881803) (xy 17.465476 -7.886517) (xy 16.992036 -7.892224) (xy 16.600496 -7.898789)
    (xy 16.302025 -7.906076) (xy 16.107792 -7.913949) (xy 16.028964 -7.922274) (xy 16.028393 -7.922598) (xy 15.97202 -7.993007)
    (xy 15.86797 -8.151439) (xy 15.7306 -8.375101) (xy 15.574268 -8.641198) (xy 15.559012 -8.66775) (xy 14.757505 -9.941295)
    (xy 13.86068 -11.135104) (xy 12.873697 -12.243995) (xy 11.801716 -13.262787) (xy 10.649898 -14.1863) (xy 9.423402 -15.009351)
    (xy 8.98525 -15.268268) (xy 8.724447 -15.422044) (xy 8.500635 -15.562903) (xy 8.339678 -15.674005) (xy 8.270875 -15.73339)
    (xy 8.253643 -15.783169) (xy 8.238893 -15.889926) (xy 8.226471 -16.061474) (xy 8.216217 -16.305627) (xy 8.207977 -16.6302)
    (xy 8.201594 -17.043006) (xy 8.196912 -17.55186) (xy 8.193773 -18.164576) (xy 8.192021 -18.888968) (xy 8.1915 -19.697137)
    (xy 8.1915 -23.5585) (xy 21.432503 -23.5585) (xy 22.622501 -22.367265))
   (layer F.Cu) (width 0.01)))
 (gr_line (start 135.636 149.606) (end 135.636 106.68) (angle 90) (layer Edge.Cuts) (width 0.1))
 (gr_line (start 138.684 152.654) (end 135.636 149.606) (angle 90) (layer Edge.Cuts) (width 0.1))
 (gr_line (start 181.356 152.654) (end 138.684 152.654) (angle 90) (layer Edge.Cuts) (width 0.1))
 (gr_line (start 184.404 149.606) (end 181.356 152.654) (angle 90) (layer Edge.Cuts) (width 0.1))
 (gr_line (start 184.404 107.188) (end 184.404 149.606) (angle 90) (layer Edge.Cuts) (width 0.1))
 (gr_line (start 181.356 104.14) (end 184.404 107.188) (angle 90) (layer Edge.Cuts) (width 0.1))
 (gr_line (start 138.176 104.14) (end 181.356 104.14) (angle 90) (layer Edge.Cuts) (width 0.1))
 (gr_line (start 135.636 106.68) (end 138.176 104.14) (angle 90) (layer Edge.Cuts) (width 0.1))
 (segment (start 141.605 150.495) (end 141.605 147.32) (width 0.25) (layer F.Cu) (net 1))
 (segment (start 141.605 147.32) (end 143.51 145.415) (width 0.25) (layer F.Cu) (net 1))
 (segment (start 158.75 148.51) (end 146.605 148.51) (width 0.25) (layer F.Cu) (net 2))
 (segment (start 146.605 148.51) (end 145.306051 147.211051) (width 0.25) (layer F.Cu) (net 2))
 (segment (start 158.75 151.05) (end 149.78 151.05) (width 0.25) (layer F.Cu) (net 3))
 (segment (start 149.78 151.05) (end 149.225 150.495) (width 0.25) (layer F.Cu) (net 3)))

